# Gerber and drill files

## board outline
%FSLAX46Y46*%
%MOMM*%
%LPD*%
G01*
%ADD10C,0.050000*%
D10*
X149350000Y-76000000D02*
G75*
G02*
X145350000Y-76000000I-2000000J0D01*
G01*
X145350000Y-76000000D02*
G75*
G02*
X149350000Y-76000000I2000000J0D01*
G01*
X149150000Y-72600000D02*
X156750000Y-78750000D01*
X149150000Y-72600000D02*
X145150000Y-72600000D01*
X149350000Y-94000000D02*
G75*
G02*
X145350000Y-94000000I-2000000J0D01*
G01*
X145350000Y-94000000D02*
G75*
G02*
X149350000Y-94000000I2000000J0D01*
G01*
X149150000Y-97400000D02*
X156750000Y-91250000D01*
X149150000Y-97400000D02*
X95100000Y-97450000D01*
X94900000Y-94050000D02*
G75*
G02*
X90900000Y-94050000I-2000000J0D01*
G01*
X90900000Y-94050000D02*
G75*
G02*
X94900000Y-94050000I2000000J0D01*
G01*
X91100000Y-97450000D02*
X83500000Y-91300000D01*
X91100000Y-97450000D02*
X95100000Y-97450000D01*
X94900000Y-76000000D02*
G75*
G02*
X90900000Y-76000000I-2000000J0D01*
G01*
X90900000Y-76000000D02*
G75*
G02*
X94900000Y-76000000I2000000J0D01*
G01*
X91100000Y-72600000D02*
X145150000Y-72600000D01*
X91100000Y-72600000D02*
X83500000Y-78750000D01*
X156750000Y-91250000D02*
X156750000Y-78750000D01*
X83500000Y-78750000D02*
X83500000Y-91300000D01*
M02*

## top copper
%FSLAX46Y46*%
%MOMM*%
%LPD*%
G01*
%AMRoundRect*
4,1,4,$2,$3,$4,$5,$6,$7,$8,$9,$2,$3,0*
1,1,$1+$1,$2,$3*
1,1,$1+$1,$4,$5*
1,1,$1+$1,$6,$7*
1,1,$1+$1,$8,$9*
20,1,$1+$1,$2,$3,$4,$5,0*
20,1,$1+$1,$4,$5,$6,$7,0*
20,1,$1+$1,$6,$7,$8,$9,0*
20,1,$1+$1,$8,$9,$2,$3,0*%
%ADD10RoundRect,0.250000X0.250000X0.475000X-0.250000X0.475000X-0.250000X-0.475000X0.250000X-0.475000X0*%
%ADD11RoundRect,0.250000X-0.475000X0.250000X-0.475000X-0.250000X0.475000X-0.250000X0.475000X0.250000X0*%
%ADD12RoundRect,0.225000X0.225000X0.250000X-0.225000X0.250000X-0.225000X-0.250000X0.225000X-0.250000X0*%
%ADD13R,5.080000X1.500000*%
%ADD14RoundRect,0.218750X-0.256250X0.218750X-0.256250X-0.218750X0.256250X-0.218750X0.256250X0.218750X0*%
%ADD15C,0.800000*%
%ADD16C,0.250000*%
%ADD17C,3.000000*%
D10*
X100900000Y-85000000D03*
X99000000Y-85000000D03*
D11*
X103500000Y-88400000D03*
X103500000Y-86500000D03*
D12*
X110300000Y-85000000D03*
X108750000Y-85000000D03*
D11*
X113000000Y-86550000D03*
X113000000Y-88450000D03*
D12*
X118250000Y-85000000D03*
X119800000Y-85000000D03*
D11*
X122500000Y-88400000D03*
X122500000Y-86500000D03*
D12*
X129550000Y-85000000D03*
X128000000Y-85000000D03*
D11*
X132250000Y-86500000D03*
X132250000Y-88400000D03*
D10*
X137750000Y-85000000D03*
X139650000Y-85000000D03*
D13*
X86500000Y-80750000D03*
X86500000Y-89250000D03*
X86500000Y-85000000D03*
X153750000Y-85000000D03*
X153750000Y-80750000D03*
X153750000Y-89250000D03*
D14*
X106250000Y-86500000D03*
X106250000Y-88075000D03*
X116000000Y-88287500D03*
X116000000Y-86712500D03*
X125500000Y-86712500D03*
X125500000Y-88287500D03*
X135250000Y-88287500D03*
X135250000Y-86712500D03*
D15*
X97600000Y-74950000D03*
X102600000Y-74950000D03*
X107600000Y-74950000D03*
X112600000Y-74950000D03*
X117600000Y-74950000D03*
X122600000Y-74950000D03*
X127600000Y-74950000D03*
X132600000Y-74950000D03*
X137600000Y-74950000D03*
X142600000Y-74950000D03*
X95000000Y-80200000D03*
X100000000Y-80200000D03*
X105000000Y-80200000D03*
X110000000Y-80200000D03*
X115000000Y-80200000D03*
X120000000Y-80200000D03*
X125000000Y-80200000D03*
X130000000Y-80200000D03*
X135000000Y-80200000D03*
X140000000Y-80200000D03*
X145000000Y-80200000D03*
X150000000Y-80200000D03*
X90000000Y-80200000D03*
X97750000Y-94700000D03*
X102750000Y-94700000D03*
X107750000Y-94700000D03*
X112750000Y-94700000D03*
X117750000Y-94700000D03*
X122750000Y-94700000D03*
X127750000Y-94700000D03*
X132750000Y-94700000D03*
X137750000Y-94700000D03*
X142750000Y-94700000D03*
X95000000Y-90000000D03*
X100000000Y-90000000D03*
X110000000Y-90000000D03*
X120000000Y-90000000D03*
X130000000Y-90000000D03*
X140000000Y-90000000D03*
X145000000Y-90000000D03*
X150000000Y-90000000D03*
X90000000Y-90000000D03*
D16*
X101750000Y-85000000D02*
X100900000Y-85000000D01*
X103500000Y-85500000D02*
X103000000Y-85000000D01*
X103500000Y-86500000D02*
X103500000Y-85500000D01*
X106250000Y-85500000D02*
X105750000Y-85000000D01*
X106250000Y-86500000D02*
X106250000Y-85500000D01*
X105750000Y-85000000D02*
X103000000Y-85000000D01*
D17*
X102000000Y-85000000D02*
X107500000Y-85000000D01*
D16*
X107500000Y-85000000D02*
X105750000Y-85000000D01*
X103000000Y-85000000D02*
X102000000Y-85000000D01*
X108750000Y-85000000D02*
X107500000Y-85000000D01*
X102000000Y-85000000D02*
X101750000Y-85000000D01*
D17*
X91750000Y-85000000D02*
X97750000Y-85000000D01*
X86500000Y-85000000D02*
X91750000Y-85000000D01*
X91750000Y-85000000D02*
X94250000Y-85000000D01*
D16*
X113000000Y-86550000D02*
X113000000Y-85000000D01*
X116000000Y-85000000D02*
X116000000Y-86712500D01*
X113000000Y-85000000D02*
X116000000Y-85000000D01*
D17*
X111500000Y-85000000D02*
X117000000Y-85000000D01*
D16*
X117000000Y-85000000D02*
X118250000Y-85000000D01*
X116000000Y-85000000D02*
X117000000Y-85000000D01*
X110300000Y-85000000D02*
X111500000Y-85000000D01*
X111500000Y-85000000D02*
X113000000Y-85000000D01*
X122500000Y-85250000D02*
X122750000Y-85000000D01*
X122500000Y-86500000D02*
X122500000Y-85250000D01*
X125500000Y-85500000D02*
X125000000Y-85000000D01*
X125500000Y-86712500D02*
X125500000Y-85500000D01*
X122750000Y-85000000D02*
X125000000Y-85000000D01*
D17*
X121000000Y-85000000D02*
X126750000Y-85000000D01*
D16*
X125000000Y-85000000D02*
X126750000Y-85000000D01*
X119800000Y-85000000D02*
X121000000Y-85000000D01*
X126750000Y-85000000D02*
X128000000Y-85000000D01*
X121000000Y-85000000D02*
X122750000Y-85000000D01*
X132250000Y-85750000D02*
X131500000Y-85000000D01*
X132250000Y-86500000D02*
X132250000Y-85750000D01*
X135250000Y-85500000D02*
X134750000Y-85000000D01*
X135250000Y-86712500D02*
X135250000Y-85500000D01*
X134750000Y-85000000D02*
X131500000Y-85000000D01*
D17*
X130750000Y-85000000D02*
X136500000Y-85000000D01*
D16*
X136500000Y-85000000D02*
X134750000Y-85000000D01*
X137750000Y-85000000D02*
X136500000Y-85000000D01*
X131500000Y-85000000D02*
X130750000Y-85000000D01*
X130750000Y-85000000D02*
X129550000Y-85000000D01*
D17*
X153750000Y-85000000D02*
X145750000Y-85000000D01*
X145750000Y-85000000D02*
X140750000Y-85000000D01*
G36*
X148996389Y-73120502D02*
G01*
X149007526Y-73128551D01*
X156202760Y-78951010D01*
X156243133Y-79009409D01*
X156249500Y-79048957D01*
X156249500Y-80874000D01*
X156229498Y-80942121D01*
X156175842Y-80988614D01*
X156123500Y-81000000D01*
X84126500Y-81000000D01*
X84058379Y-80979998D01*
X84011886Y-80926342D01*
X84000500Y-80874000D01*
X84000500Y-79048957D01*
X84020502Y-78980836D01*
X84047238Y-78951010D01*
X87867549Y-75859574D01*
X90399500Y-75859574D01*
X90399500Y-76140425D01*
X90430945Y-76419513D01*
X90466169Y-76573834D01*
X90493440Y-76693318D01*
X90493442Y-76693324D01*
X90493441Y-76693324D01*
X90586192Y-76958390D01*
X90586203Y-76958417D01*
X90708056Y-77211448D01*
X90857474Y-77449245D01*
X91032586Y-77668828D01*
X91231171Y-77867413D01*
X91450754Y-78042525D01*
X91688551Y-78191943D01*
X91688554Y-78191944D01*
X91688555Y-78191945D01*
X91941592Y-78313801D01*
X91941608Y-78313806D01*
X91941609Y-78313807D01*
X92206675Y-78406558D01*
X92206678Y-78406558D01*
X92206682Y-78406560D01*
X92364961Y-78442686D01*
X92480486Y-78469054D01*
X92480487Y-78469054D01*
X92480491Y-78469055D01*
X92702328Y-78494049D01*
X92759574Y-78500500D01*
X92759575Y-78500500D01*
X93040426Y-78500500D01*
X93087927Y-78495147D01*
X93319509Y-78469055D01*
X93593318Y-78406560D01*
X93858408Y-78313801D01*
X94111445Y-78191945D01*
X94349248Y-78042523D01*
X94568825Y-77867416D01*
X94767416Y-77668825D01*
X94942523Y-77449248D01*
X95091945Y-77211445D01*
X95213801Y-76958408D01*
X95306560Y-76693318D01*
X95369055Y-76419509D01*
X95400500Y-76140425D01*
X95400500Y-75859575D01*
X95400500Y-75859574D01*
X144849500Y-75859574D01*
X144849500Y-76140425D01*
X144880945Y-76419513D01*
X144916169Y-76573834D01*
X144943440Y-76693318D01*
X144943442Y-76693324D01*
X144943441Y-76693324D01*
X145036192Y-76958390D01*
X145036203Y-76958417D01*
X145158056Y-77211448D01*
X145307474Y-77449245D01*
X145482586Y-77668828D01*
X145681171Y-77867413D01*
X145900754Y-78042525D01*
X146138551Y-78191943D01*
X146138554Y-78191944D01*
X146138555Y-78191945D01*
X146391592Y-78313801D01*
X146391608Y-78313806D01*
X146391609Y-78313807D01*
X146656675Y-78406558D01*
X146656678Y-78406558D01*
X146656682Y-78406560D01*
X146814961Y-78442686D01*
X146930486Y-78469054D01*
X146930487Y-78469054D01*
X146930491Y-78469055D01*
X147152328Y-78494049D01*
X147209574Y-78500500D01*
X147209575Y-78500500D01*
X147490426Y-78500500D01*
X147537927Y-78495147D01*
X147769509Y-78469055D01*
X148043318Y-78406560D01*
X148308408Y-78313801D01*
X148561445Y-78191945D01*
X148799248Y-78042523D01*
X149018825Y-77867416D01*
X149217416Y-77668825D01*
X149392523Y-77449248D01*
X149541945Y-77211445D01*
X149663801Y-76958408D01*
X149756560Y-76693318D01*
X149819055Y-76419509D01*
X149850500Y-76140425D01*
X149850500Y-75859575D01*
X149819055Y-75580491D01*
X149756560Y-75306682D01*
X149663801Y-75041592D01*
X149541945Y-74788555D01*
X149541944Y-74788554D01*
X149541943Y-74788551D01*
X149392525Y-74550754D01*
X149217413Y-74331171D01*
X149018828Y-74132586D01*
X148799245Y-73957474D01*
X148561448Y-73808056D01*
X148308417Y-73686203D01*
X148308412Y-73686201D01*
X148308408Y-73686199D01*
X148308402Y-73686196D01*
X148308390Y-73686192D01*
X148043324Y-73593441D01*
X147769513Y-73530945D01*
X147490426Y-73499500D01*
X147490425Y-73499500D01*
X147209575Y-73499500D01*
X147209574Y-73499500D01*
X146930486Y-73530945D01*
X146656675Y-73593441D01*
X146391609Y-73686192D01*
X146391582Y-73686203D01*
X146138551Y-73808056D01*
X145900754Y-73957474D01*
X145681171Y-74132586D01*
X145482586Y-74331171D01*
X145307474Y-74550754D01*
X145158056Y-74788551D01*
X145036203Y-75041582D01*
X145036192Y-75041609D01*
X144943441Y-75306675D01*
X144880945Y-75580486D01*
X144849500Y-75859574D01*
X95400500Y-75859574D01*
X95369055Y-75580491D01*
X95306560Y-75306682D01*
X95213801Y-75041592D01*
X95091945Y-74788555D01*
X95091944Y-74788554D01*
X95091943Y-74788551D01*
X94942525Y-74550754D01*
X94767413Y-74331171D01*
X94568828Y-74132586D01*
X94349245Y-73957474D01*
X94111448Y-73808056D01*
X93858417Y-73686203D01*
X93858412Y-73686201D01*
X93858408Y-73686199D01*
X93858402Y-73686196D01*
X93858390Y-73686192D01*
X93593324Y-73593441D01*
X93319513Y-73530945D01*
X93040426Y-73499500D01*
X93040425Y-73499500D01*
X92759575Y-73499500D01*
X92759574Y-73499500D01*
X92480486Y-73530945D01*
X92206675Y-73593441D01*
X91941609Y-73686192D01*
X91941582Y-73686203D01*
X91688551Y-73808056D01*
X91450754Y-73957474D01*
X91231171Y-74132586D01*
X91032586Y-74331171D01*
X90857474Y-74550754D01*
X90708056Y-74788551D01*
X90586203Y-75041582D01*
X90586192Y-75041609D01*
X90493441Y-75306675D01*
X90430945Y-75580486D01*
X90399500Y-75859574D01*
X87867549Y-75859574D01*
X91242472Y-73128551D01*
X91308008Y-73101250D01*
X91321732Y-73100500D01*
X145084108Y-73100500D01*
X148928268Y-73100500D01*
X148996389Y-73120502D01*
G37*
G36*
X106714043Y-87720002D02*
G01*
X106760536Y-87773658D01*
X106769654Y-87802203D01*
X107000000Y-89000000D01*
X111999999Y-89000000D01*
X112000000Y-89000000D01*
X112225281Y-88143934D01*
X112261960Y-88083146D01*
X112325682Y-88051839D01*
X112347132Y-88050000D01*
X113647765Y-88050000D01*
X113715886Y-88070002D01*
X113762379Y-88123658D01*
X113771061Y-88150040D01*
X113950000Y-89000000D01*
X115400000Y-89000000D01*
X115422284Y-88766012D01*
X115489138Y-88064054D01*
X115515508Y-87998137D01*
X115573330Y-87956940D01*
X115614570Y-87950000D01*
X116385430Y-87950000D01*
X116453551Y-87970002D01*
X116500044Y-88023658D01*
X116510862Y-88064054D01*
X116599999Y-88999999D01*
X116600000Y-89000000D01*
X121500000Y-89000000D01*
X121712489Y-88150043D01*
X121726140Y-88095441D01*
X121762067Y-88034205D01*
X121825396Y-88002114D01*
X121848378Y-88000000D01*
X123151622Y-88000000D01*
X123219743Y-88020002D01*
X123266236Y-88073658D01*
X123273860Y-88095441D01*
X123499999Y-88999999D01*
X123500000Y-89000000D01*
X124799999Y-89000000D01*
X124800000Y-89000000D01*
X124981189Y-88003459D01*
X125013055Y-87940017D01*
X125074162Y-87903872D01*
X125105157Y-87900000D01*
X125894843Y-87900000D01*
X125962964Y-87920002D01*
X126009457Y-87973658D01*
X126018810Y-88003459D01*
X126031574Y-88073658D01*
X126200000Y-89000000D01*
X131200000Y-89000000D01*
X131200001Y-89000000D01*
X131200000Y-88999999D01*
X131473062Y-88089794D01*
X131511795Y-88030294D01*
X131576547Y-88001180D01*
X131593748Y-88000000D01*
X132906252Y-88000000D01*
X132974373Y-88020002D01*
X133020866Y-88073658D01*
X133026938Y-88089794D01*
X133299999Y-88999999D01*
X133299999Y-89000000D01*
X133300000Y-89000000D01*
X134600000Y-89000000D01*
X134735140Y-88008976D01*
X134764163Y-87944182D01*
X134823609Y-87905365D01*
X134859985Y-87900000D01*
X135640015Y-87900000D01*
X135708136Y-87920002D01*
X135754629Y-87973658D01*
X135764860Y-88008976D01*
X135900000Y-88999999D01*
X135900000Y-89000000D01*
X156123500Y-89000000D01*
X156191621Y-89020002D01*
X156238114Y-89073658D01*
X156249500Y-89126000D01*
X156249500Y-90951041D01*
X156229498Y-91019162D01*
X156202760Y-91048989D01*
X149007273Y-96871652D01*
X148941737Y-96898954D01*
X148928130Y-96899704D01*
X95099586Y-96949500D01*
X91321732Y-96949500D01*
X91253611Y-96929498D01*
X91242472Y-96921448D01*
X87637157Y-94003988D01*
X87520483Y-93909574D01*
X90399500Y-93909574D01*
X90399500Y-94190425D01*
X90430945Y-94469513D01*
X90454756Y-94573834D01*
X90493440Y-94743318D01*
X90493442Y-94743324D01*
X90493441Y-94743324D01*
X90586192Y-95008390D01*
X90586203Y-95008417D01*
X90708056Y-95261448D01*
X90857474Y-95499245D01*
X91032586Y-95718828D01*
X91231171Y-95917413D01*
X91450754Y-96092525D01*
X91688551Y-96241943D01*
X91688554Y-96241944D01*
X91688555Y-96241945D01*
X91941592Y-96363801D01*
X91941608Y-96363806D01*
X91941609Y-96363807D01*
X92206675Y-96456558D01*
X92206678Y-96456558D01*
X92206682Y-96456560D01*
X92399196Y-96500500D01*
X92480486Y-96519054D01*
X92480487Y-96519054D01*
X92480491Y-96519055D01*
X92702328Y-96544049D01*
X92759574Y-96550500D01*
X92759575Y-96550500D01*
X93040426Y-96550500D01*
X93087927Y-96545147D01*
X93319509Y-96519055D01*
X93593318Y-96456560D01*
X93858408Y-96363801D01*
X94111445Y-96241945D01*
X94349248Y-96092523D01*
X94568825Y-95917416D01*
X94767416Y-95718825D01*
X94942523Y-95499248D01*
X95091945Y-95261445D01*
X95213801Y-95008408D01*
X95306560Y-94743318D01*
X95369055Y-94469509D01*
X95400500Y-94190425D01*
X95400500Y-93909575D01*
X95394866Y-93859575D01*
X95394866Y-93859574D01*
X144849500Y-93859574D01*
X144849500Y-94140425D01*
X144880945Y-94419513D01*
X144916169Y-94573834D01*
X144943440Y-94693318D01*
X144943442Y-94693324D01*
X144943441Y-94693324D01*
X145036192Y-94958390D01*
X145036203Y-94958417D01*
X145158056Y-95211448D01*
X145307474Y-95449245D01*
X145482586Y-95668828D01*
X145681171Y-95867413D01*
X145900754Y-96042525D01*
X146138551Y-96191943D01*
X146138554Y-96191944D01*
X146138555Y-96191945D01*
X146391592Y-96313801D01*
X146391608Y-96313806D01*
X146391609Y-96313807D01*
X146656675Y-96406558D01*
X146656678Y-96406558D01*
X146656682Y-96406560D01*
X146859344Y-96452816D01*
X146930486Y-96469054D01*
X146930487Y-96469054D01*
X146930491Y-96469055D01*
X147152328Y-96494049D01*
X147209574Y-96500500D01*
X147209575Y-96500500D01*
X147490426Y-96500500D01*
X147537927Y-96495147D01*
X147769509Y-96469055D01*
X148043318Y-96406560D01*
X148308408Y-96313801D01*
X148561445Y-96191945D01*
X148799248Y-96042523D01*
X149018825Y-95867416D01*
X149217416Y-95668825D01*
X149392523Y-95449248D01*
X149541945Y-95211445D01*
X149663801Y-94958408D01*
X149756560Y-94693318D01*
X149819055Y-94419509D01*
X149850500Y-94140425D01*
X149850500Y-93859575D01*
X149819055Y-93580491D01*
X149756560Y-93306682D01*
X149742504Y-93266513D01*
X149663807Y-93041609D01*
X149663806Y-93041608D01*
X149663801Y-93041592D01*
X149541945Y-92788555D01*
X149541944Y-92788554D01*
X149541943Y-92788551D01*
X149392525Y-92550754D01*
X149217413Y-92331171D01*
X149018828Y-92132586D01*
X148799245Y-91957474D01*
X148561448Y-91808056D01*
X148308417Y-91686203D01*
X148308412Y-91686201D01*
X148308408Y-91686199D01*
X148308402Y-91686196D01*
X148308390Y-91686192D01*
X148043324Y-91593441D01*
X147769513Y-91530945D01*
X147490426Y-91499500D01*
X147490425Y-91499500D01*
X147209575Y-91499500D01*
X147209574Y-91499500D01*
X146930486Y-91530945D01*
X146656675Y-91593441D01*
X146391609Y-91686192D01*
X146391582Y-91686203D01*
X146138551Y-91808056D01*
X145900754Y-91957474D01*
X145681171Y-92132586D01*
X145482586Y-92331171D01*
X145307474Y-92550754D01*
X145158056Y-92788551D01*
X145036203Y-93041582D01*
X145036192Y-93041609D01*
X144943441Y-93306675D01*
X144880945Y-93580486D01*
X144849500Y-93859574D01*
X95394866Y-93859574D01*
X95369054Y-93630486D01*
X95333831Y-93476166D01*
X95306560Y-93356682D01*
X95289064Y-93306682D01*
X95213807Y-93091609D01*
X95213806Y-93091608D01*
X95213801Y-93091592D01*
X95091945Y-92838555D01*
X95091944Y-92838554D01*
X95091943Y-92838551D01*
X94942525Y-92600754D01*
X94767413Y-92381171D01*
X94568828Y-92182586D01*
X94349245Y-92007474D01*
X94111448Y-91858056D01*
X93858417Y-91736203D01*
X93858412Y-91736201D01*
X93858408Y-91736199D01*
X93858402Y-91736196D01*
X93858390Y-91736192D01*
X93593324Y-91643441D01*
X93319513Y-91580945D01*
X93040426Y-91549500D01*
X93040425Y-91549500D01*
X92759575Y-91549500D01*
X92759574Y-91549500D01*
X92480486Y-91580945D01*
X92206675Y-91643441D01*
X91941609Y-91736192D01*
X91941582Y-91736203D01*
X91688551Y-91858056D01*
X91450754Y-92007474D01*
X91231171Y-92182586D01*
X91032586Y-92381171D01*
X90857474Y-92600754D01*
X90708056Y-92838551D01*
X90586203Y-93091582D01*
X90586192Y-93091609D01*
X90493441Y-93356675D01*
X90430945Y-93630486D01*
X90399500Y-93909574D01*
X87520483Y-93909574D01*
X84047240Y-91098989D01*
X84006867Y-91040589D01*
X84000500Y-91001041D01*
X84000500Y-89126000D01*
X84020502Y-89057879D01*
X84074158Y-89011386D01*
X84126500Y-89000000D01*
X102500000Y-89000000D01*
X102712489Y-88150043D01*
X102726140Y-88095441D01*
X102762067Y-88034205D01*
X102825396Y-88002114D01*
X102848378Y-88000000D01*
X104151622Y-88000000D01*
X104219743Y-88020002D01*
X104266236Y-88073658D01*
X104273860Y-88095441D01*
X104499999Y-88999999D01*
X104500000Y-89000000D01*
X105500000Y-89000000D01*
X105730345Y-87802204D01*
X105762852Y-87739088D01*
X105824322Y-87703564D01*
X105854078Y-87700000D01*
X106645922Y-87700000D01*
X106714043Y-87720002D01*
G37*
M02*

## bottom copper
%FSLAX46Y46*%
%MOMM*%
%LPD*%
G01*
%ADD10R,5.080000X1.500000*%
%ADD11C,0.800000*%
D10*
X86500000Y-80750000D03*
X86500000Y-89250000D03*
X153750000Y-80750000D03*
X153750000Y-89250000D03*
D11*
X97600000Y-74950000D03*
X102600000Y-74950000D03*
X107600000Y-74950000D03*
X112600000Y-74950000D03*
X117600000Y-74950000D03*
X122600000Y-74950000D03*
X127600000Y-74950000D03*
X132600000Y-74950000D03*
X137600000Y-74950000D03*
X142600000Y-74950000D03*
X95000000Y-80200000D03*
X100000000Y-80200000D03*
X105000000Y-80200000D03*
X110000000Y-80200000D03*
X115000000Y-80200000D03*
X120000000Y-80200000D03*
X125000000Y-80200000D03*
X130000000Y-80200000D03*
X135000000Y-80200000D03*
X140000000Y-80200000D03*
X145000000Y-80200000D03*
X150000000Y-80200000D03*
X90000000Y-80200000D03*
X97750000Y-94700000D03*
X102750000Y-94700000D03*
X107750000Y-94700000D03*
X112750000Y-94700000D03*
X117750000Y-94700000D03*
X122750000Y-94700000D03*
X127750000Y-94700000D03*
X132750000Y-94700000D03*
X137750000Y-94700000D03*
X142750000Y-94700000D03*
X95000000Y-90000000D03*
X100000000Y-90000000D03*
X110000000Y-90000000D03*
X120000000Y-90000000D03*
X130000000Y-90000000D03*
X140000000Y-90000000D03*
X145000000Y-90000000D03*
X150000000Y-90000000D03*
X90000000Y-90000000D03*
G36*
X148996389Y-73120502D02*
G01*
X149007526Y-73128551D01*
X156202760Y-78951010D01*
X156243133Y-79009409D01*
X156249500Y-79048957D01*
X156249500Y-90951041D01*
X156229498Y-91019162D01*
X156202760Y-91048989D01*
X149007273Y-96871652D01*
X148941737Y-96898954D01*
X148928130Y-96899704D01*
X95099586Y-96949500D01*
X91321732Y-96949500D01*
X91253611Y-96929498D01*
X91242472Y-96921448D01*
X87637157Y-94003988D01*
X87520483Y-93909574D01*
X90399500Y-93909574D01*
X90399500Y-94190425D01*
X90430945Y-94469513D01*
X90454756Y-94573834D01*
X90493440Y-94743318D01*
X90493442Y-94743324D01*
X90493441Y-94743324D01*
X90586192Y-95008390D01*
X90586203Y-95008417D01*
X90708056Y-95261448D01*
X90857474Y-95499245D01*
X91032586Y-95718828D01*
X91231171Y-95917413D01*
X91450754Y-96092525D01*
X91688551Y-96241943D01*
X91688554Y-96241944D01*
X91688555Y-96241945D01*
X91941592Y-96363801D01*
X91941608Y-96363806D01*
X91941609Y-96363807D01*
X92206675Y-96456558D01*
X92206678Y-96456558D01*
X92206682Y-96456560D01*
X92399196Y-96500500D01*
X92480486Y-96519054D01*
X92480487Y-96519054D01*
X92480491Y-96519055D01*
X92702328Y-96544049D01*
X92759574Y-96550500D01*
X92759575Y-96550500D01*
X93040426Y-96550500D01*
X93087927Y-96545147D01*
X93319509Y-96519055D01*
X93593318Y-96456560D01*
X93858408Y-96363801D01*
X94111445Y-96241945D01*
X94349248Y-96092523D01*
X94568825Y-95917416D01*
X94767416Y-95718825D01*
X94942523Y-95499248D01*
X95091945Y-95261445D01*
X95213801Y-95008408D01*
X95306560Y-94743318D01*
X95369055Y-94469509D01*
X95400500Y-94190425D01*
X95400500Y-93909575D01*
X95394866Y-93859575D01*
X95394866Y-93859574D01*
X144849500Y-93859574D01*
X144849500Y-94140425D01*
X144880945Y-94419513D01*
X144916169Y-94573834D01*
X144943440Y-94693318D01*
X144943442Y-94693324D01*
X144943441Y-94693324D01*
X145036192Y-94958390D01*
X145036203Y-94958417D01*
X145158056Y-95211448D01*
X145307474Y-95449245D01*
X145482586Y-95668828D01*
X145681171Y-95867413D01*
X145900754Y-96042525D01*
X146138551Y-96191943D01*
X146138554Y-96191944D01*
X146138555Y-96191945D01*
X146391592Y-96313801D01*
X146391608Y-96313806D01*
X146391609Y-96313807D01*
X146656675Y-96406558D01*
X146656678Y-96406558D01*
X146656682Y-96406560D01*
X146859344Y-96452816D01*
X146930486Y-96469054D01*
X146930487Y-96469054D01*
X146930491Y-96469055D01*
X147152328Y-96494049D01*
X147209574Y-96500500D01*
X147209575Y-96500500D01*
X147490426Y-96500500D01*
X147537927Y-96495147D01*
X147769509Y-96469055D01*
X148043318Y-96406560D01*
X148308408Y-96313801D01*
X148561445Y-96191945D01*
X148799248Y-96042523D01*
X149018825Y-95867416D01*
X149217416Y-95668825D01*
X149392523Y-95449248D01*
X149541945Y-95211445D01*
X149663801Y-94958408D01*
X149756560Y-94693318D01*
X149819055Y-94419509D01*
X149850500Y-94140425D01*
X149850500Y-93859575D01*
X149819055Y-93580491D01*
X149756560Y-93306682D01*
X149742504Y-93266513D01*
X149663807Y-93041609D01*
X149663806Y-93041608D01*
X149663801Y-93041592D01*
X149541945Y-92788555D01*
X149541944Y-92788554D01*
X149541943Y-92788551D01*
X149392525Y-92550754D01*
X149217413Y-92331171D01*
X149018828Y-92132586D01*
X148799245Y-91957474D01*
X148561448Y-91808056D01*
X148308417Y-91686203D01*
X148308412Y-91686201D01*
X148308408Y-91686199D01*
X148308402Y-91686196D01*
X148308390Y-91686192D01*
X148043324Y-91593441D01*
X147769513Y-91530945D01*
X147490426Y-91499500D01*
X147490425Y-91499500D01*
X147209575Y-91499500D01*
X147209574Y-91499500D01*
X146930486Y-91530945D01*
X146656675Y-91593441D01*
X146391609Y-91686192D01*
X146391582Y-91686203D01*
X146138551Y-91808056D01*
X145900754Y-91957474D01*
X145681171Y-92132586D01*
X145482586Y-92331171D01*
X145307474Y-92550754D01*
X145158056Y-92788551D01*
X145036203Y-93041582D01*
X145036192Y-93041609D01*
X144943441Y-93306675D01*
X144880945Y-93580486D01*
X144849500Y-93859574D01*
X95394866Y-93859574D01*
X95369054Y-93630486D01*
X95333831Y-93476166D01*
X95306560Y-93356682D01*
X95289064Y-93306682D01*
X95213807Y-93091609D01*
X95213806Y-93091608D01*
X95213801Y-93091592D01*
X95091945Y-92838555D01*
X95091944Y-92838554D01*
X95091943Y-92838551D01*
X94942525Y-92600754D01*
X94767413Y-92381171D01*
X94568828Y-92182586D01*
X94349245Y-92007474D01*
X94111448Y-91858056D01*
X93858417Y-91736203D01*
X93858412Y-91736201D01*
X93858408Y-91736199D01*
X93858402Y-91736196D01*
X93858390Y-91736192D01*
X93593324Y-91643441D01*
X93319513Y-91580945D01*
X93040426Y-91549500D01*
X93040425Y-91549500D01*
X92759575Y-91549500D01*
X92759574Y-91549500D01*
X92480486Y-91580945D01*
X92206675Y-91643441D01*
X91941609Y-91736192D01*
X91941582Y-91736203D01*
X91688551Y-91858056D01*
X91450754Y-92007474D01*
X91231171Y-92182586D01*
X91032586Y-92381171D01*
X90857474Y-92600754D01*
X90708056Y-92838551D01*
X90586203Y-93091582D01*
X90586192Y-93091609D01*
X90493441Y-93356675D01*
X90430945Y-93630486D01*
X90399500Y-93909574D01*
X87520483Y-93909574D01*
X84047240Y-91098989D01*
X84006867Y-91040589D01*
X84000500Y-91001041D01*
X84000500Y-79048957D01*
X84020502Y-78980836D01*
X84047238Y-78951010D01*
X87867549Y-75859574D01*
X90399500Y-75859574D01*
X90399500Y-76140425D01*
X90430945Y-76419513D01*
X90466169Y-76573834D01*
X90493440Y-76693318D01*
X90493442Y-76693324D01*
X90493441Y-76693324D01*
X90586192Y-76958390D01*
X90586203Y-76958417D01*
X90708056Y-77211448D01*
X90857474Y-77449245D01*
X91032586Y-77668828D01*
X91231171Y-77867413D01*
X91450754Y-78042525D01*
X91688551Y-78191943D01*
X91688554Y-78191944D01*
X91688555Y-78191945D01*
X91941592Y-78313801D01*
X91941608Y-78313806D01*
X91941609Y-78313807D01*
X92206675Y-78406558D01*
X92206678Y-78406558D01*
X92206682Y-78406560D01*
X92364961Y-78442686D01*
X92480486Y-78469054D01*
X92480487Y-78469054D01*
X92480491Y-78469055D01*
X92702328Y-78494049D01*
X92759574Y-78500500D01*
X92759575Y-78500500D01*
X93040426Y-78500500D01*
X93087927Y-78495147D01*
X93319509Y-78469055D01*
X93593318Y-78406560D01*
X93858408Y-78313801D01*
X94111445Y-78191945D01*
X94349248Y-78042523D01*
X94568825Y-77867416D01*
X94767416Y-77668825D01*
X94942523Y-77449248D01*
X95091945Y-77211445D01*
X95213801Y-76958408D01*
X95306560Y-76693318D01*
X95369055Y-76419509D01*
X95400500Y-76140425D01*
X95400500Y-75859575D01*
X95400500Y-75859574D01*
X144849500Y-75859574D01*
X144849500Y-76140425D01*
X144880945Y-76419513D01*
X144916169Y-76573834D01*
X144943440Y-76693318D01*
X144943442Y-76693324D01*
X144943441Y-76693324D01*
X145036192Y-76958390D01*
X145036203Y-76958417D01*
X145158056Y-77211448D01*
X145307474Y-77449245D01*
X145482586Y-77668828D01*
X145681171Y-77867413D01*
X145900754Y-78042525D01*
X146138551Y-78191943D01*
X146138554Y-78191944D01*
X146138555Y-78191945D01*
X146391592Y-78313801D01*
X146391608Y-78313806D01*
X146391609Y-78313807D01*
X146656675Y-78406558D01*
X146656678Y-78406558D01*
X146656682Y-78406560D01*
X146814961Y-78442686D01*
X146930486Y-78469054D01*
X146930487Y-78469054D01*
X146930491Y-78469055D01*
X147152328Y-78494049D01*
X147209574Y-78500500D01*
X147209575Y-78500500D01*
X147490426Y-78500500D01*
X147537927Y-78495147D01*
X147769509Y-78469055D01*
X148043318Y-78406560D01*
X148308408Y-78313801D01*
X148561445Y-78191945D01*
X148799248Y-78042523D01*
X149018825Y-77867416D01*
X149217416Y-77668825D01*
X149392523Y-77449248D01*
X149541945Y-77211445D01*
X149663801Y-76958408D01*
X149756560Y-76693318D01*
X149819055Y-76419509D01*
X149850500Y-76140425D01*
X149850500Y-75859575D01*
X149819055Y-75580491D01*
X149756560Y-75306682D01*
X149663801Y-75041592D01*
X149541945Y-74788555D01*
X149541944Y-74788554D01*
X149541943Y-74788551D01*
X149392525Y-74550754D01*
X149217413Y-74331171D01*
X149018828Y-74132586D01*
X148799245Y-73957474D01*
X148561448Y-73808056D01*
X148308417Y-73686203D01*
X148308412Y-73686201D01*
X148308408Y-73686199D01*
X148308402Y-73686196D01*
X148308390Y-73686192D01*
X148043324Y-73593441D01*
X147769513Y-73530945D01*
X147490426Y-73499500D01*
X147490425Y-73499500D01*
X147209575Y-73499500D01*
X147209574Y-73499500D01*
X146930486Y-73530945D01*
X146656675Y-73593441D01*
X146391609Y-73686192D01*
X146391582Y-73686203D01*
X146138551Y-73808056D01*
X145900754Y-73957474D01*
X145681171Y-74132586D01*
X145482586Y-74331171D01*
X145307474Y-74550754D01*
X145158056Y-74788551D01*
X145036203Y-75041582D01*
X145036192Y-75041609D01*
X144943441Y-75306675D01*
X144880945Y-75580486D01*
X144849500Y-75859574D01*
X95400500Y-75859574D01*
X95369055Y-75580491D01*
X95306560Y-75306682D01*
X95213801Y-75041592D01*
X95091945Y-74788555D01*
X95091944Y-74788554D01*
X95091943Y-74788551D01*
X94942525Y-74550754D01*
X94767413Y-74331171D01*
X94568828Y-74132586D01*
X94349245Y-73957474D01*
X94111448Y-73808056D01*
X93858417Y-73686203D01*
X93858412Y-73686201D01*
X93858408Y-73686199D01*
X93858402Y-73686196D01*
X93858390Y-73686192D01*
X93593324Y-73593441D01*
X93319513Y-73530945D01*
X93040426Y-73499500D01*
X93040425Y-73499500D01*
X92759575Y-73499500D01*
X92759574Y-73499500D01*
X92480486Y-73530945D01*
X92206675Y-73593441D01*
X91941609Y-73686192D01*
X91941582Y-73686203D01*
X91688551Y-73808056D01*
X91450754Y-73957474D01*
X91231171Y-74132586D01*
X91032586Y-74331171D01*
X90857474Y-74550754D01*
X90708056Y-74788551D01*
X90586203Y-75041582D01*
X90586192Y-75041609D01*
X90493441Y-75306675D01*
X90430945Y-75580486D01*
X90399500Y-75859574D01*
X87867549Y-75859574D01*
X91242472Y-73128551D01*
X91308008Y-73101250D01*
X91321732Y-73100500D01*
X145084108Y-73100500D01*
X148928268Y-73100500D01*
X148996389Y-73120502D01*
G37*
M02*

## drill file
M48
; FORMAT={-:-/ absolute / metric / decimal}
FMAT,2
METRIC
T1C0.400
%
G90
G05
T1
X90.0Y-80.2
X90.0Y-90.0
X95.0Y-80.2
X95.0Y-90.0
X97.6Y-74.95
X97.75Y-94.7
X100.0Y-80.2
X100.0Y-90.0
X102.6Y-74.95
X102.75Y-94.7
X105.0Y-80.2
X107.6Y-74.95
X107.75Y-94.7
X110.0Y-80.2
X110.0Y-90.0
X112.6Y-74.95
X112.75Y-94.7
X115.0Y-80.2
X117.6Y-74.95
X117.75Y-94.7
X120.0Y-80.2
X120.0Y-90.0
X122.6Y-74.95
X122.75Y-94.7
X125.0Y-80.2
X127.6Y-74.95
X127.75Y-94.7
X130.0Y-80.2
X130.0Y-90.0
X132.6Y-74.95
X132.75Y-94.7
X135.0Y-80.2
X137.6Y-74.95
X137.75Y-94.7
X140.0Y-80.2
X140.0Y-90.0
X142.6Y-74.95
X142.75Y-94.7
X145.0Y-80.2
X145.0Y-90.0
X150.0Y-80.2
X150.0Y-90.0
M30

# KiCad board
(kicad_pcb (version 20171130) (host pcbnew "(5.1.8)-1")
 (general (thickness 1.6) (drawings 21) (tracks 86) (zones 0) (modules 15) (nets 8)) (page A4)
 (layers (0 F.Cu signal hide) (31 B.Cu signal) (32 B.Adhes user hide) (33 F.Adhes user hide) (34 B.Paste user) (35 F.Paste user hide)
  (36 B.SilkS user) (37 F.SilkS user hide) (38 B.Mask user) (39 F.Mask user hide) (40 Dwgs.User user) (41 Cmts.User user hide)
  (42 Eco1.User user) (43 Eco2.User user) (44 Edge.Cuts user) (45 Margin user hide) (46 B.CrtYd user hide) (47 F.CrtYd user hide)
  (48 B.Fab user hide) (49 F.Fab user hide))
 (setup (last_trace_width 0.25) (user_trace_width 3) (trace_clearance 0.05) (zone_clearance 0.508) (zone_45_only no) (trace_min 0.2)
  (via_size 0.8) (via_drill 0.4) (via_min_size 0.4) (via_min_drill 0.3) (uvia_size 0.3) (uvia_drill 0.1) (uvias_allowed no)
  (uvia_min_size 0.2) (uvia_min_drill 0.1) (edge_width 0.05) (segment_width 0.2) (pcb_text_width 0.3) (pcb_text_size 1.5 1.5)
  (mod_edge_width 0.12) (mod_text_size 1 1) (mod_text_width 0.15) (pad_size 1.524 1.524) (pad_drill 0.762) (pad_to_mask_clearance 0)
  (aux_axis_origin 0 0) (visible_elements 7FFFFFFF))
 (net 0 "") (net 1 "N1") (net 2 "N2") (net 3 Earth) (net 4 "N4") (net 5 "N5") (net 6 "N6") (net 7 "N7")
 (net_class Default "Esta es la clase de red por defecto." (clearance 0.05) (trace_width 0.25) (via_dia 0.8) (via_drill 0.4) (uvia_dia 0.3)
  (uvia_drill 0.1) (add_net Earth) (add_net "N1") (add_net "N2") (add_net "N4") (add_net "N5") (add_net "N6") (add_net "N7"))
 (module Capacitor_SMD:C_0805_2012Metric (layer F.Cu) (at 99.95 85 180)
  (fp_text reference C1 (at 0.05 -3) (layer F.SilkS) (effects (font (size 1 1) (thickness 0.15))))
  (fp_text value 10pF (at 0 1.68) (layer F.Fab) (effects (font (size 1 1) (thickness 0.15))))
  (pad 1 smd roundrect (at -0.95 0 180) (size 1 1.45) (layers F.Cu F.Paste F.Mask) (roundrect_rratio 0.25) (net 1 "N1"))
  (pad 2 smd roundrect (at 0.95 0 180) (size 1 1.45) (layers F.Cu F.Paste F.Mask) (roundrect_rratio 0.25) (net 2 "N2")))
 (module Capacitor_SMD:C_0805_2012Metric (layer F.Cu) (at 103.5 87.45 270)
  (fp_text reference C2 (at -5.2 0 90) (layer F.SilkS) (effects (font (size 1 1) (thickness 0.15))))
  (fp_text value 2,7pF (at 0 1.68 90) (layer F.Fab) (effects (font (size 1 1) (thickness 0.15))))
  (pad 2 smd roundrect (at 0.95 0 270) (size 1 1.45) (layers F.Cu F.Paste F.Mask) (roundrect_rratio 0.25) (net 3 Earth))
  (pad 1 smd roundrect (at -0.95 0 270) (size 1 1.45) (layers F.Cu F.Paste F.Mask) (roundrect_rratio 0.25) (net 1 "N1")))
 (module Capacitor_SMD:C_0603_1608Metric (layer F.Cu) (at 109.525 85 180)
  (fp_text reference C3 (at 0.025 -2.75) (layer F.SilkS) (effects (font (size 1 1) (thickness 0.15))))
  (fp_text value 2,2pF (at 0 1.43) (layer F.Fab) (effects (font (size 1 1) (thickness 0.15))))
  (pad 1 smd roundrect (at -0.775 0 180) (size 0.9 0.95) (layers F.Cu F.Paste F.Mask) (roundrect_rratio 0.25) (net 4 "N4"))
  (pad 2 smd roundrect (at 0.775 0 180) (size 0.9 0.95) (layers F.Cu F.Paste F.Mask) (roundrect_rratio 0.25) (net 1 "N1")))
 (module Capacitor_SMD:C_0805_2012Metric (layer F.Cu) (at 113 87.5 270)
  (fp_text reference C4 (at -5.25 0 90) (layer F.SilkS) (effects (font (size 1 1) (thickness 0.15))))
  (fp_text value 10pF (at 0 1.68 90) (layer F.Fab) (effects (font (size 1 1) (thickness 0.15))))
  (pad 1 smd roundrect (at -0.95 0 270) (size 1 1.45) (layers F.Cu F.Paste F.Mask) (roundrect_rratio 0.25) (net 4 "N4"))
  (pad 2 smd roundrect (at 0.95 0 270) (size 1 1.45) (layers F.Cu F.Paste F.Mask) (roundrect_rratio 0.25) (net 3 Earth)))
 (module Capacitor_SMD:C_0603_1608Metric (layer F.Cu) (at 119.025 85 180)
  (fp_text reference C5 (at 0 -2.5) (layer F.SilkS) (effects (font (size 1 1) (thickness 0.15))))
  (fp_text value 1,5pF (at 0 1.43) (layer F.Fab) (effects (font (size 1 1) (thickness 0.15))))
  (pad 2 smd roundrect (at 0.775 0 180) (size 0.9 0.95) (layers F.Cu F.Paste F.Mask) (roundrect_rratio 0.25) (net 4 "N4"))
  (pad 1 smd roundrect (at -0.775 0 180) (size 0.9 0.95) (layers F.Cu F.Paste F.Mask) (roundrect_rratio 0.25) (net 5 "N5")))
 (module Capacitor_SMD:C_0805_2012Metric (layer F.Cu) (at 122.5 87.45 270)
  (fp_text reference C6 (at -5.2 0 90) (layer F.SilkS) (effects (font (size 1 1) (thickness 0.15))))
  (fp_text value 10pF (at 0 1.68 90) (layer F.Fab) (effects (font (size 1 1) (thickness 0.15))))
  (pad 2 smd roundrect (at 0.95 0 270) (size 1 1.45) (layers F.Cu F.Paste F.Mask) (roundrect_rratio 0.25) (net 3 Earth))
  (pad 1 smd roundrect (at -0.95 0 270) (size 1 1.45) (layers F.Cu F.Paste F.Mask) (roundrect_rratio 0.25) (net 5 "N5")))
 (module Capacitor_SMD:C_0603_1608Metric (layer F.Cu) (at 128.775 85 180)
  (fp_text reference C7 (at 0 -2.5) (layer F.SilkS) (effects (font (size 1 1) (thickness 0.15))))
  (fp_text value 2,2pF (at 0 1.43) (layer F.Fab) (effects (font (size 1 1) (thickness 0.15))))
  (pad 1 smd roundrect (at -0.775 0 180) (size 0.9 0.95) (layers F.Cu F.Paste F.Mask) (roundrect_rratio 0.25) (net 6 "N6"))
  (pad 2 smd roundrect (at 0.775 0 180) (size 0.9 0.95) (layers F.Cu F.Paste F.Mask) (roundrect_rratio 0.25) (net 5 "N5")))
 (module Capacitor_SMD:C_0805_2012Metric (layer F.Cu) (at 132.25 87.45 270)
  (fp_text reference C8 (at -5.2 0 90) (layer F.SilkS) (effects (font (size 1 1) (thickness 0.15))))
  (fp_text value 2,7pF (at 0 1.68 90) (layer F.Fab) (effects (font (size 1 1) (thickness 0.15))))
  (pad 1 smd roundrect (at -0.95 0 270) (size 1 1.45) (layers F.Cu F.Paste F.Mask) (roundrect_rratio 0.25) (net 6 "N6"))
  (pad 2 smd roundrect (at 0.95 0 270) (size 1 1.45) (layers F.Cu F.Paste F.Mask) (roundrect_rratio 0.25) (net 3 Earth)))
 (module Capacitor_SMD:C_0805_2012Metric (layer F.Cu) (at 138.7 85 180)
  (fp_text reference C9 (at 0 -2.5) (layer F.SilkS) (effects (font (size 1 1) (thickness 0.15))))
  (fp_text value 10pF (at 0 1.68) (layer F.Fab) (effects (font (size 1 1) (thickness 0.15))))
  (pad 2 smd roundrect (at 0.95 0 180) (size 1 1.45) (layers F.Cu F.Paste F.Mask) (roundrect_rratio 0.25) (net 6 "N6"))
  (pad 1 smd roundrect (at -0.95 0 180) (size 1 1.45) (layers F.Cu F.Paste F.Mask) (roundrect_rratio 0.25) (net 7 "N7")))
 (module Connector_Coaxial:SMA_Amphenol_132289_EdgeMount (layer F.Cu) (at 86.5 85 180)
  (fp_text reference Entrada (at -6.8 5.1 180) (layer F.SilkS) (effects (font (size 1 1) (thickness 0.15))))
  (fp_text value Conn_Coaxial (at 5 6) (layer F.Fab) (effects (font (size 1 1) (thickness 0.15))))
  (pad 2 smd rect (at 0 4.25 270) (size 1.5 5.08) (layers B.Cu B.Paste B.Mask) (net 3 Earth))
  (pad 2 smd rect (at 0 -4.25 270) (size 1.5 5.08) (layers B.Cu B.Paste B.Mask) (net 3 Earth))
  (pad 2 smd rect (at 0 4.25 270) (size 1.5 5.08) (layers F.Cu F.Paste F.Mask) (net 3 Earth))
  (pad 2 smd rect (at 0 -4.25 270) (size 1.5 5.08) (layers F.Cu F.Paste F.Mask) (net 3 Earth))
  (pad 1 smd rect (at 0 0 270) (size 1.5 5.08) (layers F.Cu F.Paste F.Mask) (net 2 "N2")))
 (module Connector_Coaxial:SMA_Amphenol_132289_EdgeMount (layer F.Cu) (at 153.75 85)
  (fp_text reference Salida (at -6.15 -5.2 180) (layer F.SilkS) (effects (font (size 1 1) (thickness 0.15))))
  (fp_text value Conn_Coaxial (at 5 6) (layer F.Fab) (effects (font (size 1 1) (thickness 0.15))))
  (pad 1 smd rect (at 0 0 90) (size 1.5 5.08) (layers F.Cu F.Paste F.Mask) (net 7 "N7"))
  (pad 2 smd rect (at 0 -4.25 90) (size 1.5 5.08) (layers F.Cu F.Paste F.Mask) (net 3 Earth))
  (pad 2 smd rect (at 0 4.25 90) (size 1.5 5.08) (layers F.Cu F.Paste F.Mask) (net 3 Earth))
  (pad 2 smd rect (at 0 -4.25 90) (size 1.5 5.08) (layers B.Cu B.Paste B.Mask) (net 3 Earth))
  (pad 2 smd rect (at 0 4.25 90) (size 1.5 5.08) (layers B.Cu B.Paste B.Mask) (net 3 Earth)))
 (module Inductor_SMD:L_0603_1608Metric (layer F.Cu) (at 106.25 87.2875 270)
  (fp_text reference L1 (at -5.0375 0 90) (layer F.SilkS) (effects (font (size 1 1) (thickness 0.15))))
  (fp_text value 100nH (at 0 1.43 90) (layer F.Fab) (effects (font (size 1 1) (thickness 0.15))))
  (pad 1 smd roundrect (at -0.7875 0 270) (size 0.875 0.95) (layers F.Cu F.Paste F.Mask) (roundrect_rratio 0.25) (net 1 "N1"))
  (pad 2 smd roundrect (at 0.7875 0 270) (size 0.875 0.95) (layers F.Cu F.Paste F.Mask) (roundrect_rratio 0.25) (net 3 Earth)))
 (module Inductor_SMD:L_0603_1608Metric (layer F.Cu) (at 116 87.5 270)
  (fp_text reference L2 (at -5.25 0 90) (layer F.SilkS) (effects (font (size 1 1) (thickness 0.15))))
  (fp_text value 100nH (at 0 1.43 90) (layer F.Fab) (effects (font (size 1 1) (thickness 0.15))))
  (pad 2 smd roundrect (at 0.7875 0 270) (size 0.875 0.95) (layers F.Cu F.Paste F.Mask) (roundrect_rratio 0.25) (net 3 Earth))
  (pad 1 smd roundrect (at -0.7875 0 270) (size 0.875 0.95) (layers F.Cu F.Paste F.Mask) (roundrect_rratio 0.25) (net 4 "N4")))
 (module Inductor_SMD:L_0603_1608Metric (layer F.Cu) (at 125.5 87.5 270)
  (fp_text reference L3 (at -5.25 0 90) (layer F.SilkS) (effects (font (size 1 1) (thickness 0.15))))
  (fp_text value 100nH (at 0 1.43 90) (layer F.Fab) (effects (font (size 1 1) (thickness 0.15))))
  (pad 1 smd roundrect (at -0.7875 0 270) (size 0.875 0.95) (layers F.Cu F.Paste F.Mask) (roundrect_rratio 0.25) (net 5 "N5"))
  (pad 2 smd roundrect (at 0.7875 0 270) (size 0.875 0.95) (layers F.Cu F.Paste F.Mask) (roundrect_rratio 0.25) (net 3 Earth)))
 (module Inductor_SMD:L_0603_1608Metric (layer F.Cu) (at 135.25 87.5 270)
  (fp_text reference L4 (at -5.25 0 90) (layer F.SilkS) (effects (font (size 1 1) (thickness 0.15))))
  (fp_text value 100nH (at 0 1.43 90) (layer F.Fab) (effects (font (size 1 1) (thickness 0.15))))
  (pad 2 smd roundrect (at 0.7875 0 270) (size 0.875 0.95) (layers F.Cu F.Paste F.Mask) (roundrect_rratio 0.25) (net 3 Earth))
  (pad 1 smd roundrect (at -0.7875 0 270) (size 0.875 0.95) (layers F.Cu F.Paste F.Mask) (roundrect_rratio 0.25) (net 6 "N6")))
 (gr_circle (center 147.35 76) (end 145.35 76) (layer Edge.Cuts) (width 0.05))
 (gr_line (start 149.15 72.6) (end 156.75 78.75) (layer Edge.Cuts) (width 0.05))
 (gr_line (start 149.15 72.6) (end 145.15 72.6) (layer Edge.Cuts) (width 0.05))
 (gr_circle (center 147.35 94) (end 145.35 94) (layer Edge.Cuts) (width 0.05))
 (gr_line (start 149.15 97.4) (end 156.75 91.25) (layer Edge.Cuts) (width 0.05))
 (gr_line (start 149.15 97.4) (end 95.1 97.45) (layer Edge.Cuts) (width 0.05))
 (gr_circle (center 92.9 94.05) (end 94.9 94.05) (layer Edge.Cuts) (width 0.05))
 (gr_line (start 91.1 97.45) (end 83.5 91.3) (layer Edge.Cuts) (width 0.05))
 (gr_line (start 91.1 97.45) (end 95.1 97.45) (layer Edge.Cuts) (width 0.05))
 (gr_circle (center 92.9 76) (end 94.9 76) (layer Edge.Cuts) (width 0.05))
 (gr_line (start 91.1 72.6) (end 145.15 72.6) (layer Edge.Cuts) (width 0.05))
 (gr_line (start 91.1 72.6) (end 83.5 78.75) (layer Edge.Cuts) (width 0.05))
 (gr_line (start 156.75 91.25) (end 156.75 78.75) (layer Edge.Cuts) (width 0.05))
 (gr_line (start 83.5 78.75) (end 83.5 91.3) (layer Edge.Cuts) (width 0.05))
 (segment (start 101.75 85) (end 100.9 85) (width 0.25) (layer F.Cu) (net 1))
 (segment (start 103.5 85.5) (end 103 85) (width 0.25) (layer F.Cu) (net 1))
 (segment (start 103.5 86.5) (end 103.5 85.5) (width 0.25) (layer F.Cu) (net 1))
 (segment (start 106.25 85.5) (end 105.75 85) (width 0.25) (layer F.Cu) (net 1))
 (segment (start 106.25 86.5) (end 106.25 85.5) (width 0.25) (layer F.Cu) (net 1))
 (segment (start 105.75 85) (end 103 85) (width 0.25) (layer F.Cu) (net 1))
 (segment (start 102 85) (end 107.5 85) (width 3) (layer F.Cu) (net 1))
 (segment (start 107.5 85) (end 105.75 85) (width 0.25) (layer F.Cu) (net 1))
 (segment (start 103 85) (end 102 85) (width 0.25) (layer F.Cu) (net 1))
 (segment (start 108.75 85) (end 107.5 85) (width 0.25) (layer F.Cu) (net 1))
 (segment (start 102 85) (end 101.75 85) (width 0.25) (layer F.Cu) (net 1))
 (segment (start 91.75 85) (end 97.75 85) (width 3) (layer F.Cu) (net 2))
 (segment (start 86.5 85) (end 91.75 85) (width 3) (layer F.Cu) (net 2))
 (segment (start 91.75 85) (end 94.25 85) (width 3) (layer F.Cu) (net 2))
 (via (at 97.6 74.95) (size 0.8) (drill 0.4) (layers F.Cu B.Cu) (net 3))
 (via (at 102.6 74.95) (size 0.8) (drill 0.4) (layers F.Cu B.Cu) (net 3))
 (via (at 107.6 74.95) (size 0.8) (drill 0.4) (layers F.Cu B.Cu) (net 3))
 (via (at 112.6 74.95) (size 0.8) (drill 0.4) (layers F.Cu B.Cu) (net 3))
 (via (at 117.6 74.95) (size 0.8) (drill 0.4) (layers F.Cu B.Cu) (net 3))
 (via (at 122.6 74.95) (size 0.8) (drill 0.4) (layers F.Cu B.Cu) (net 3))
 (via (at 127.6 74.95) (size 0.8) (drill 0.4) (layers F.Cu B.Cu) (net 3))
 (via (at 132.6 74.95) (size 0.8) (drill 0.4) (layers F.Cu B.Cu) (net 3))
 (via (at 137.6 74.95) (size 0.8) (drill 0.4) (layers F.Cu B.Cu) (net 3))
 (via (at 142.6 74.95) (size 0.8) (drill 0.4) (layers F.Cu B.Cu) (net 3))
 (via (at 95 80.2) (size 0.8) (drill 0.4) (layers F.Cu B.Cu) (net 3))
 (via (at 100 80.2) (size 0.8) (drill 0.4) (layers F.Cu B.Cu) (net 3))
 (via (at 105 80.2) (size 0.8) (drill 0.4) (layers F.Cu B.Cu) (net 3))
 (via (at 110 80.2) (size 0.8) (drill 0.4) (layers F.Cu B.Cu) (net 3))
 (via (at 115 80.2) (size 0.8) (drill 0.4) (layers F.Cu B.Cu) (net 3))
 (via (at 120 80.2) (size 0.8) (drill 0.4) (layers F.Cu B.Cu) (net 3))
 (via (at 125 80.2) (size 0.8) (drill 0.4) (layers F.Cu B.Cu) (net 3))
 (via (at 130 80.2) (size 0.8) (drill 0.4) (layers F.Cu B.Cu) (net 3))
 (via (at 135 80.2) (size 0.8) (drill 0.4) (layers F.Cu B.Cu) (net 3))
 (via (at 140 80.2) (size 0.8) (drill 0.4) (layers F.Cu B.Cu) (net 3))
 (via (at 145 80.2) (size 0.8) (drill 0.4) (layers F.Cu B.Cu) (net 3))
 (via (at 150 80.2) (size 0.8) (drill 0.4) (layers F.Cu B.Cu) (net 3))
 (via (at 90 80.2) (size 0.8) (drill 0.4) (layers F.Cu B.Cu) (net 3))
 (via (at 97.75 94.7) (size 0.8) (drill 0.4) (layers F.Cu B.Cu) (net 3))
 (via (at 102.75 94.7) (size 0.8) (drill 0.4) (layers F.Cu B.Cu) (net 3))
 (via (at 107.75 94.7) (size 0.8) (drill 0.4) (layers F.Cu B.Cu) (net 3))
 (via (at 112.75 94.7) (size 0.8) (drill 0.4) (layers F.Cu B.Cu) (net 3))
 (via (at 117.75 94.7) (size 0.8) (drill 0.4) (layers F.Cu B.Cu) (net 3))
 (via (at 122.75 94.7) (size 0.8) (drill 0.4) (layers F.Cu B.Cu) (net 3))
 (via (at 127.75 94.7) (size 0.8) (drill 0.4) (layers F.Cu B.Cu) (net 3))
 (via (at 132.75 94.7) (size 0.8) (drill 0.4) (layers F.Cu B.Cu) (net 3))
 (via (at 137.75 94.7) (size 0.8) (drill 0.4) (layers F.Cu B.Cu) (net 3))
 (via (at 142.75 94.7) (size 0.8) (drill 0.4) (layers F.Cu B.Cu) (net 3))
 (via (at 95 90) (size 0.8) (drill 0.4) (layers F.Cu B.Cu) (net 3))
 (via (at 100 90) (size 0.8) (drill 0.4) (layers F.Cu B.Cu) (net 3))
 (via (at 110 90) (size 0.8) (drill 0.4) (layers F.Cu B.Cu) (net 3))
 (via (at 120 90) (size 0.8) (drill 0.4) (layers F.Cu B.Cu) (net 3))
 (via (at 130 90) (size 0.8) (drill 0.4) (layers F.Cu B.Cu) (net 3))
 (via (at 140 90) (size 0.8) (drill 0.4) (layers F.Cu B.Cu) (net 3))
 (via (at 145 90) (size 0.8) (drill 0.4) (layers F.Cu B.Cu) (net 3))
 (via (at 150 90) (size 0.8) (drill 0.4) (layers F.Cu B.Cu) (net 3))
 (via (at 90 90) (size 0.8) (drill 0.4) (layers F.Cu B.Cu) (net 3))
 (segment (start 113 86.55) (end 113 85) (width 0.25) (layer F.Cu) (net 4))
 (segment (start 116 85) (end 116 86.7125) (width 0.25) (layer F.Cu) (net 4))
 (segment (start 113 85) (end 116 85) (width 0.25) (layer F.Cu) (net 4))
 (segment (start 111.5 85) (end 117 85) (width 3) (layer F.Cu) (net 4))
 (segment (start 117 85) (end 118.25 85) (width 0.25) (layer F.Cu) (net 4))
 (segment (start 116 85) (end 117 85) (width 0.25) (layer F.Cu) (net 4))
 (segment (start 110.3 85) (end 111.5 85) (width 0.25) (layer F.Cu) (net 4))
 (segment (start 111.5 85) (end 113 85) (width 0.25) (layer F.Cu) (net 4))
 (segment (start 122.5 85.25) (end 122.75 85) (width 0.25) (layer F.Cu) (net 5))
 (segment (start 122.5 86.5) (end 122.5 85.25) (width 0.25) (layer F.Cu) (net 5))
 (segment (start 125.5 85.5) (end 125 85) (width 0.25) (layer F.Cu) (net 5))
 (segment (start 125.5 86.7125) (end 125.5 85.5) (width 0.25) (layer F.Cu) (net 5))
 (segment (start 122.75 85) (end 125 85) (width 0.25) (layer F.Cu) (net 5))
 (segment (start 121 85) (end 126.75 85) (width 3) (layer F.Cu) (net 5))
 (segment (start 125 85) (end 126.75 85) (width 0.25) (layer F.Cu) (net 5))
 (segment (start 119.8 85) (end 121 85) (width 0.25) (layer F.Cu) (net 5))
 (segment (start 126.75 85) (end 128 85) (width 0.25) (layer F.Cu) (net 5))
 (segment (start 121 85) (end 122.75 85) (width 0.25) (layer F.Cu) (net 5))
 (segment (start 132.25 85.75) (end 131.5 85) (width 0.25) (layer F.Cu) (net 6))
 (segment (start 132.25 86.5) (end 132.25 85.75) (width 0.25) (layer F.Cu) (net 6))
 (segment (start 135.25 85.5) (end 134.75 85) (width 0.25) (layer F.Cu) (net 6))
 (segment (start 135.25 86.7125) (end 135.25 85.5) (width 0.25) (layer F.Cu) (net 6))
 (segment (start 134.75 85) (end 131.5 85) (width 0.25) (layer F.Cu) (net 6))
 (segment (start 130.75 85) (end 136.5 85) (width 3) (layer F.Cu) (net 6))
 (segment (start 136.5 85) (end 134.75 85) (width 0.25) (layer F.Cu) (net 6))
 (segment (start 137.75 85) (end 136.5 85) (width 0.25) (layer F.Cu) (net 6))
 (segment (start 131.5 85) (end 130.75 85) (width 0.25) (layer F.Cu) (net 6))
 (segment (start 130.75 85) (end 129.55 85) (width 0.25) (layer F.Cu) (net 6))
 (segment (start 153.75 85) (end 145.75 85) (width 3) (layer F.Cu) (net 7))
 (segment (start 145.75 85) (end 140.75 85) (width 3) (layer F.Cu) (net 7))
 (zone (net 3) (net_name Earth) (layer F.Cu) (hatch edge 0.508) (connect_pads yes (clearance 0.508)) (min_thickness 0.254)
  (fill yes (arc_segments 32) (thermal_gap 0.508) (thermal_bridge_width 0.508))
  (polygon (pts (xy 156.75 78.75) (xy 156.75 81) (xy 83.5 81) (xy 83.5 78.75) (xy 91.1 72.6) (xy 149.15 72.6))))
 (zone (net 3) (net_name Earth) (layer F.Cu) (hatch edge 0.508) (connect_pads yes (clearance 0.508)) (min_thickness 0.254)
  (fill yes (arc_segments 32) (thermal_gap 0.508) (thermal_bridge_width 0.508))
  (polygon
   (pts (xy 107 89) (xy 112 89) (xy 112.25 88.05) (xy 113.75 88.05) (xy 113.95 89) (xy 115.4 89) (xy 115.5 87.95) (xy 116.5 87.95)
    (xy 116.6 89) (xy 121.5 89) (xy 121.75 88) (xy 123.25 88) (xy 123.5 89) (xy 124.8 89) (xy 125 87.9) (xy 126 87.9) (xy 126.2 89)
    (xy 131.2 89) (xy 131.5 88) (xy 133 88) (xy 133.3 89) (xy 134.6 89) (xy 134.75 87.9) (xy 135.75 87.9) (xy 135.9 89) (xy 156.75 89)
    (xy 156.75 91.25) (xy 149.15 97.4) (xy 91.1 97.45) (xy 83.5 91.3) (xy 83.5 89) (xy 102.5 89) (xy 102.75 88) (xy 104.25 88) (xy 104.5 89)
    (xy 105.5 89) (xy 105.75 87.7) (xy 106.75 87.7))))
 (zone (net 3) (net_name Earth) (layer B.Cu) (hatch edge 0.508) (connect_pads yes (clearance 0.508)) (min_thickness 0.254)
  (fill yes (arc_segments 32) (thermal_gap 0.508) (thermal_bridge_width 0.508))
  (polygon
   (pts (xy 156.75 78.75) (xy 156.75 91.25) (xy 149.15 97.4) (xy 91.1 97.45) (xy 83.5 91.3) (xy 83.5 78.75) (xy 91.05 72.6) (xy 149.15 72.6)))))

